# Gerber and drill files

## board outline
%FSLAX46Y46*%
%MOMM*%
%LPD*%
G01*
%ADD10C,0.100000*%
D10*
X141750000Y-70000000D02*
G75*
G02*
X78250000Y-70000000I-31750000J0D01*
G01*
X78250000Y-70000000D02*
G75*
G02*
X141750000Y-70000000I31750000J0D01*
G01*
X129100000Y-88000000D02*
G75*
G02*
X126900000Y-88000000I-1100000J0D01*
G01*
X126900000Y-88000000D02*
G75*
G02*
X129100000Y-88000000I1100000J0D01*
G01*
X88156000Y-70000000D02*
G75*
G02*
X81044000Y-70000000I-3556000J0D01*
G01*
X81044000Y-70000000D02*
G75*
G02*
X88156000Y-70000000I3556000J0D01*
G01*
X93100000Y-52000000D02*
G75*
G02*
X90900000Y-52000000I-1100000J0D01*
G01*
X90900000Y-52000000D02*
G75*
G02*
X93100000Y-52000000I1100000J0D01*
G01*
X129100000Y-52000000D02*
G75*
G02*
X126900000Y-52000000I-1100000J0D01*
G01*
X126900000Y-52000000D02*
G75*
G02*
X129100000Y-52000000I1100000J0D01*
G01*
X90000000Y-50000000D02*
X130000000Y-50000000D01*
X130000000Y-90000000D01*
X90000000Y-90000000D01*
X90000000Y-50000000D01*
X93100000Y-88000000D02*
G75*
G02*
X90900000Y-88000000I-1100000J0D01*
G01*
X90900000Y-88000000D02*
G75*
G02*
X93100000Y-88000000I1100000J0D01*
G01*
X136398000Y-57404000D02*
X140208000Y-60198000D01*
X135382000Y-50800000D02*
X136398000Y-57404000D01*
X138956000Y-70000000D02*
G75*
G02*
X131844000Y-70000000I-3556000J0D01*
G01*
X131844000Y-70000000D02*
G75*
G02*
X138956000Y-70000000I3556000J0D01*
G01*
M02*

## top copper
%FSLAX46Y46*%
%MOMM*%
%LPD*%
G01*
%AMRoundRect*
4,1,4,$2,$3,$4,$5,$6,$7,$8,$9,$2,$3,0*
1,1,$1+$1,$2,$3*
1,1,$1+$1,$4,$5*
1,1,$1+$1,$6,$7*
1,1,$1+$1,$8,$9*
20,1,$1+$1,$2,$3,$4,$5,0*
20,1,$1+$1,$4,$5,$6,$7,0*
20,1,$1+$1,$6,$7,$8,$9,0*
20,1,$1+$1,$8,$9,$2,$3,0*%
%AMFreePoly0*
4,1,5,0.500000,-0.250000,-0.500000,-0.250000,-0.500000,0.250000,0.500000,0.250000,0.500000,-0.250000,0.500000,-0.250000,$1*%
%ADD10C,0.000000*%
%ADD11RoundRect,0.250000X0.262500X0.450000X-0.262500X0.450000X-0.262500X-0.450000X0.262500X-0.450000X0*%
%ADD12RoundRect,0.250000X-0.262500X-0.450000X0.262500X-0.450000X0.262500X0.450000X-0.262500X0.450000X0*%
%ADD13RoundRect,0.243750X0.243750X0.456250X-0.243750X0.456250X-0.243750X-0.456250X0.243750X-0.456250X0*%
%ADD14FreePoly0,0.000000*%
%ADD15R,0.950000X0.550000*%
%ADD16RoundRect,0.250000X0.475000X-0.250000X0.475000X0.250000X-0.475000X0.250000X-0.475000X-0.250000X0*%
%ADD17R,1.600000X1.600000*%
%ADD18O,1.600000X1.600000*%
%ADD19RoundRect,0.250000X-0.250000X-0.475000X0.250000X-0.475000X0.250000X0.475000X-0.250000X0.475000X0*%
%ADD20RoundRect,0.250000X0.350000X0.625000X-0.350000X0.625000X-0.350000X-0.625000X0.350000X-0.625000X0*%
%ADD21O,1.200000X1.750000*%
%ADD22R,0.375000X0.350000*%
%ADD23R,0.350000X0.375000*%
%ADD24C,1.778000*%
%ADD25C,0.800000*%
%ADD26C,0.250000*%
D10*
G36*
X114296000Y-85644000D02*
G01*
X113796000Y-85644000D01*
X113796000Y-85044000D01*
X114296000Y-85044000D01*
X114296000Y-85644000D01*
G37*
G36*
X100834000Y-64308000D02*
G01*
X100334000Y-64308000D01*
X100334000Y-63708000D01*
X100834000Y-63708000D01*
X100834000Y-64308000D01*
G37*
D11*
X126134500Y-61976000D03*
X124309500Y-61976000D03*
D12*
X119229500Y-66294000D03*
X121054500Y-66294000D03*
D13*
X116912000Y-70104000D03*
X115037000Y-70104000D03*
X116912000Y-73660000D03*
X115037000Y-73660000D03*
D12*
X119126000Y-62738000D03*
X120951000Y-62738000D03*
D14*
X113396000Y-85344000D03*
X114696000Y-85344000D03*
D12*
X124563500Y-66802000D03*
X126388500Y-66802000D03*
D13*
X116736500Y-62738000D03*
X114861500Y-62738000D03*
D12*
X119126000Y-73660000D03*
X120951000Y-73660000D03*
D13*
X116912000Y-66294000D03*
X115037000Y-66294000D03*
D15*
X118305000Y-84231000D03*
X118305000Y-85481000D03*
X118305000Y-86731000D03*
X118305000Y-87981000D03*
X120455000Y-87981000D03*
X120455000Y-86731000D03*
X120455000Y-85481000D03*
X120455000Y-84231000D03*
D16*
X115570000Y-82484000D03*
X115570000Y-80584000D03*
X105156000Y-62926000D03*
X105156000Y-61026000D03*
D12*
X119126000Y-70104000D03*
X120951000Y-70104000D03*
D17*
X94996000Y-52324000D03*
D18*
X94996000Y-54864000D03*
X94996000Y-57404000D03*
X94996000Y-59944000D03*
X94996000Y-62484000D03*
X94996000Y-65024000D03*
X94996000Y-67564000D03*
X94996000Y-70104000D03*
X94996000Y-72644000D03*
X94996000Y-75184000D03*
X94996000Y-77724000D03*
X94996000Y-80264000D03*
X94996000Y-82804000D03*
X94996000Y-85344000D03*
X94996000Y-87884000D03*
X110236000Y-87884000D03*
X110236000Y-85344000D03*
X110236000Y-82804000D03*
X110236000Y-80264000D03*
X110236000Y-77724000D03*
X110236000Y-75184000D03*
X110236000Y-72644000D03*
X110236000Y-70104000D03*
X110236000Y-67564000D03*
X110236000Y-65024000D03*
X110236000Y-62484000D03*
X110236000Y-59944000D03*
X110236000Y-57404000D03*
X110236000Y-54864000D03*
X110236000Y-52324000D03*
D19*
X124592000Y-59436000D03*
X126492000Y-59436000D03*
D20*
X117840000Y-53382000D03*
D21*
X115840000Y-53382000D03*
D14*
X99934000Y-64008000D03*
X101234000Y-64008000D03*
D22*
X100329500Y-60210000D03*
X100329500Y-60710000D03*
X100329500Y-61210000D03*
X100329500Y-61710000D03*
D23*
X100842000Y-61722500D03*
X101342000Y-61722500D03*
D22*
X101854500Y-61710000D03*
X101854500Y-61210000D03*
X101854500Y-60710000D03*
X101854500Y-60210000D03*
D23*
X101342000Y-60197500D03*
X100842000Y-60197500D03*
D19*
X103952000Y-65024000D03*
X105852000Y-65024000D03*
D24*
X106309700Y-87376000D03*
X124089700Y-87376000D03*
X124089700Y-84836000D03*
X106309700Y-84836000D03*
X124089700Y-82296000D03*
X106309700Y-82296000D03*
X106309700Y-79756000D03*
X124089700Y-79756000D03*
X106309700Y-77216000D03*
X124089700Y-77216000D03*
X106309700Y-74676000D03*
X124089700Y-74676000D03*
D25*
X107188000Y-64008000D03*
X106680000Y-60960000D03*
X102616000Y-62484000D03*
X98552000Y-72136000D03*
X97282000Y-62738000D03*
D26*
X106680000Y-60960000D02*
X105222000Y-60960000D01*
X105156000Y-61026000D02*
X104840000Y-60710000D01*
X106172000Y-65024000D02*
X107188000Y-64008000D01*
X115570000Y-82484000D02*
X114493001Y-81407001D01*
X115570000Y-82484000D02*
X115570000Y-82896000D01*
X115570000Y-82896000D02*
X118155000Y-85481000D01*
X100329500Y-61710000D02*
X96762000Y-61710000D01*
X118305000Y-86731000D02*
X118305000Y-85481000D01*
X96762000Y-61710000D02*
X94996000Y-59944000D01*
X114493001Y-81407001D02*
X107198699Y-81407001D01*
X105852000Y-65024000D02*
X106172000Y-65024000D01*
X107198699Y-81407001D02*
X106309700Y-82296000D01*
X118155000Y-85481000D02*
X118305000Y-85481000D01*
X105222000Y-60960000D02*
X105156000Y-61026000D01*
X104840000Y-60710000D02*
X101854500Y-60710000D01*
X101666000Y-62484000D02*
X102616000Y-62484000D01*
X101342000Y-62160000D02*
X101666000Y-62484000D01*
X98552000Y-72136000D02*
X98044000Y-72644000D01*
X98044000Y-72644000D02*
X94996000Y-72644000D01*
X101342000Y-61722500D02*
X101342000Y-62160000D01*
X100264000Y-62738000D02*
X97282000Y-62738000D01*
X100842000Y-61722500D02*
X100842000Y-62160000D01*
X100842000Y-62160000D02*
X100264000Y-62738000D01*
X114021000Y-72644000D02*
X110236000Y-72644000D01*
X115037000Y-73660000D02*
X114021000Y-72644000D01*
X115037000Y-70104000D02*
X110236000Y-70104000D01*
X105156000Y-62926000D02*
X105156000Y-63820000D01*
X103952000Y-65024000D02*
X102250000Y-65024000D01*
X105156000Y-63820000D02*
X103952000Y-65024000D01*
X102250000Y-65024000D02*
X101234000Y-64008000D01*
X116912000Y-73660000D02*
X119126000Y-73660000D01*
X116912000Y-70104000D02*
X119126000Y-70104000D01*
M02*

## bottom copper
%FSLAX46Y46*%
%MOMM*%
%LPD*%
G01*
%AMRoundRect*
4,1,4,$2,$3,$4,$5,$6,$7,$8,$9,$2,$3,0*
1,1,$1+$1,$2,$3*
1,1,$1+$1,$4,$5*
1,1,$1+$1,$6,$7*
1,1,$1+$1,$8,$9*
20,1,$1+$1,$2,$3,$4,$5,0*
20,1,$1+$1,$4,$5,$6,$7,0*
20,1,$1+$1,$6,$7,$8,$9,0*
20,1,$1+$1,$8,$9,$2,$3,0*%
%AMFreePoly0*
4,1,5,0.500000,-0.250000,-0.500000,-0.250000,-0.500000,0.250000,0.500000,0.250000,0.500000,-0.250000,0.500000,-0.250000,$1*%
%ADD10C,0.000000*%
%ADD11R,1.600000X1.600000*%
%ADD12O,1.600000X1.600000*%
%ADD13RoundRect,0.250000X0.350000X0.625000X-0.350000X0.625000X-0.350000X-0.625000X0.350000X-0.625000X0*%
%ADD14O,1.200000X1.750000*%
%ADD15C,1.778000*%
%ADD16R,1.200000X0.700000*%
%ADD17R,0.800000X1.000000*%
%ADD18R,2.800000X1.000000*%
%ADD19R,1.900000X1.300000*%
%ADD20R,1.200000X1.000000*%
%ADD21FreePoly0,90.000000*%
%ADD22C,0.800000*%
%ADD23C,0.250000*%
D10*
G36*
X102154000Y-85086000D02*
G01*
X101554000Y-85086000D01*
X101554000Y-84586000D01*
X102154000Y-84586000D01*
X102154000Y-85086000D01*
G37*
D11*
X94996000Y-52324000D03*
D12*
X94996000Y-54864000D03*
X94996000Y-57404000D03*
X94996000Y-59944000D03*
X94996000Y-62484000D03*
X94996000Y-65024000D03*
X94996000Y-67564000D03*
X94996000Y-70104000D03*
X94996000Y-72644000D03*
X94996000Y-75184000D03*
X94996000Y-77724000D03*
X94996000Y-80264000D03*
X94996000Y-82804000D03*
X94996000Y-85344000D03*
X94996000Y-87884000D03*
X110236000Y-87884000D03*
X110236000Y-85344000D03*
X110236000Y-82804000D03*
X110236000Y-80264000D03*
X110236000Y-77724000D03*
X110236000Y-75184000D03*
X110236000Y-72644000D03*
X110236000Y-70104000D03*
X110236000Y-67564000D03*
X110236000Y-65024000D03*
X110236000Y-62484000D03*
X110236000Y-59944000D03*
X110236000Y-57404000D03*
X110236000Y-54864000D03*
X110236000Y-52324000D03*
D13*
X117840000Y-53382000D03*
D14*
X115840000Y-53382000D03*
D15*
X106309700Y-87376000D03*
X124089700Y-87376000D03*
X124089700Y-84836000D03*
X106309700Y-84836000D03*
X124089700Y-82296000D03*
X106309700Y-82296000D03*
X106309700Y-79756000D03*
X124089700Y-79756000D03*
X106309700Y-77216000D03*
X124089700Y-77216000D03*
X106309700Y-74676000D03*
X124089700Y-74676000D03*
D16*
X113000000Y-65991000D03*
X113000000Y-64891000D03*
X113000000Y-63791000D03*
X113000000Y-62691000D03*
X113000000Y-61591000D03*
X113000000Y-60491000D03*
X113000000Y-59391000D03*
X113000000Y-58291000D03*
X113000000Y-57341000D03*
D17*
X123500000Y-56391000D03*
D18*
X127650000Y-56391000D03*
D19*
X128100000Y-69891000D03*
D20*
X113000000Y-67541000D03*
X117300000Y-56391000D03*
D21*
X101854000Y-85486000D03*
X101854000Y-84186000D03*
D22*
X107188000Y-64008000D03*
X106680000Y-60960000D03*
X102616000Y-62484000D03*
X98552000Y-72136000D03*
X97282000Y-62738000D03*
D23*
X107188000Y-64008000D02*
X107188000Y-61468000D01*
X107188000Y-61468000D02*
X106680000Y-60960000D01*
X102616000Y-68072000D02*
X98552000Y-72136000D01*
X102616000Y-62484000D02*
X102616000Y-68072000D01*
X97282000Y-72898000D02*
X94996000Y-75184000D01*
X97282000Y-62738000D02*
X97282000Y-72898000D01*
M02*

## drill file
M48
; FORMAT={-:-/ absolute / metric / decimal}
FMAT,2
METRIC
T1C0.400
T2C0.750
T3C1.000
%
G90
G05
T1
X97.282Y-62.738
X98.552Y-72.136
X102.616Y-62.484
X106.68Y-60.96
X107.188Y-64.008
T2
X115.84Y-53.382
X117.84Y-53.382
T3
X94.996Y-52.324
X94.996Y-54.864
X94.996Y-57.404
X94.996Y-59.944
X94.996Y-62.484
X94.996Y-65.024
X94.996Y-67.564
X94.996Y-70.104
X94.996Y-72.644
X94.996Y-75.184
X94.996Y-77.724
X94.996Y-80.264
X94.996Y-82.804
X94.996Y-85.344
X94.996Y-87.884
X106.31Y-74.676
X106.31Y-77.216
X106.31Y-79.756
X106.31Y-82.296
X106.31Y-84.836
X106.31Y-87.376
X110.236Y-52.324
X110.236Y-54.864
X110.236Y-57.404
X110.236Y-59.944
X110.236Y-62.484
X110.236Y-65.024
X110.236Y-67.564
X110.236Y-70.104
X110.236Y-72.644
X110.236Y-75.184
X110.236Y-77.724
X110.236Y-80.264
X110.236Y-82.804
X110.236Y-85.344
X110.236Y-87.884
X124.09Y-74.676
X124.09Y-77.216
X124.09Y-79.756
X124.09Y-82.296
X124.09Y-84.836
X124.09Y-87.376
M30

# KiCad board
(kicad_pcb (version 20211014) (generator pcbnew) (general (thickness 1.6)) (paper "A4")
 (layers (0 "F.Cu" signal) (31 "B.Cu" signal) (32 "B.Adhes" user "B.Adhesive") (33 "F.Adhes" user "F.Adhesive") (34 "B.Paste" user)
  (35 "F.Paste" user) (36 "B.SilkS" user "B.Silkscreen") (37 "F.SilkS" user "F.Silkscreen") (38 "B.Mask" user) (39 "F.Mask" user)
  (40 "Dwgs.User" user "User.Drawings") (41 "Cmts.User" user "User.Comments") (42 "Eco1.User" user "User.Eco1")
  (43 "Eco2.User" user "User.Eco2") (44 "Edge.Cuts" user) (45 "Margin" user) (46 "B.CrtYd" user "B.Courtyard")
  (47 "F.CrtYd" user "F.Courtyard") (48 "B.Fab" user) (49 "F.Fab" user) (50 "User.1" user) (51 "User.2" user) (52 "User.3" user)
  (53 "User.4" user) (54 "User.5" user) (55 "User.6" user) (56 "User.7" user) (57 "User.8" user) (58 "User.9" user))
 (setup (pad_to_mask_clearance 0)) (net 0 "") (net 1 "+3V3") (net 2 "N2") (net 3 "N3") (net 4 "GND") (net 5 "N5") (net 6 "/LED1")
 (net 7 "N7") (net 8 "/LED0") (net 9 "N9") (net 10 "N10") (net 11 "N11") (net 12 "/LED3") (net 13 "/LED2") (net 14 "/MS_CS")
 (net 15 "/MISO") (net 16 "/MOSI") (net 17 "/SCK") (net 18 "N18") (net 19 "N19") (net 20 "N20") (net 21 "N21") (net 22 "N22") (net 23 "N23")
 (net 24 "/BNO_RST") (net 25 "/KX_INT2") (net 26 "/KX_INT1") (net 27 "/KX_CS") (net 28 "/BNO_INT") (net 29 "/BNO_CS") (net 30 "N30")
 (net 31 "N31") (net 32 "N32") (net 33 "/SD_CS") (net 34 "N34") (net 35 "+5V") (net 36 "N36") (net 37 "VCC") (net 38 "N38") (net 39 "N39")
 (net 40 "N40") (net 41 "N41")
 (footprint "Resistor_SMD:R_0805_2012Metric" (layer "F.Cu") (at 125.222 61.976 180)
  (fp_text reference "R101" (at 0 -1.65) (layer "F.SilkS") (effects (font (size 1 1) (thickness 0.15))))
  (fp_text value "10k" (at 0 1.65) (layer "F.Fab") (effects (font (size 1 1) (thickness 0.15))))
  (pad "1" smd roundrect (at -0.9125 0 180) (size 1.025 1.4) (layers "F.Cu" "F.Paste" "F.Mask") (roundrect_rratio 0.243902) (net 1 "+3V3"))
  (pad "2" smd roundrect (at 0.9125 0 180) (size 1.025 1.4) (layers "F.Cu" "F.Paste" "F.Mask") (roundrect_rratio 0.243902) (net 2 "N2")))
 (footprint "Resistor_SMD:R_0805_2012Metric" (layer "F.Cu") (at 120.142 66.294)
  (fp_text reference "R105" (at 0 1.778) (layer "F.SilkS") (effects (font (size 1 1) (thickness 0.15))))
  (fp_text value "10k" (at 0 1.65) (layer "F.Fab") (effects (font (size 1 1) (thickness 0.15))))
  (pad "1" smd roundrect (at -0.9125 0) (size 1.025 1.4) (layers "F.Cu" "F.Paste" "F.Mask") (roundrect_rratio 0.243902) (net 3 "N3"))
  (pad "2" smd roundrect (at 0.9125 0) (size 1.025 1.4) (layers "F.Cu" "F.Paste" "F.Mask") (roundrect_rratio 0.243902) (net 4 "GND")))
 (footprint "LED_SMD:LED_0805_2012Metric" (layer "F.Cu") (at 115.9745 70.104 180)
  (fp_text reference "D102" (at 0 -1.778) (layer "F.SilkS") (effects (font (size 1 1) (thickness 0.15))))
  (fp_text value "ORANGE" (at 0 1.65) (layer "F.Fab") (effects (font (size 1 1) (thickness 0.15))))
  (pad "1" smd roundrect (at -0.9375 0 180) (size 0.975 1.4) (layers "F.Cu" "F.Paste" "F.Mask") (roundrect_rratio 0.25) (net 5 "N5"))
  (pad "2" smd roundrect (at 0.9375 0 180) (size 0.975 1.4) (layers "F.Cu" "F.Paste" "F.Mask") (roundrect_rratio 0.25) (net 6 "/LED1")))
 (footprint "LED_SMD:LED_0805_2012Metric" (layer "F.Cu") (at 115.9745 73.66 180)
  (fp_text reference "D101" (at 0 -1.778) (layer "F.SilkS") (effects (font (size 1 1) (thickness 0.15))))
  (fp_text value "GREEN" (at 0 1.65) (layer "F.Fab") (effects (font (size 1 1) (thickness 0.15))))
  (pad "1" smd roundrect (at -0.9375 0 180) (size 0.975 1.4) (layers "F.Cu" "F.Paste" "F.Mask") (roundrect_rratio 0.25) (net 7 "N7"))
  (pad "2" smd roundrect (at 0.9375 0 180) (size 0.975 1.4) (layers "F.Cu" "F.Paste" "F.Mask") (roundrect_rratio 0.25) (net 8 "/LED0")))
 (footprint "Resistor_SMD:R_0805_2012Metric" (layer "F.Cu") (at 120.0385 62.738)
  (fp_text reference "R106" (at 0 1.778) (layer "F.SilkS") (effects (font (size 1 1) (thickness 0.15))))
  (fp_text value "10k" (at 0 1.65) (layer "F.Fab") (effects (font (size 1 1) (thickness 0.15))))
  (pad "1" smd roundrect (at -0.9125 0) (size 1.025 1.4) (layers "F.Cu" "F.Paste" "F.Mask") (roundrect_rratio 0.243902) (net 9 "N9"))
  (pad "2" smd roundrect (at 0.9125 0) (size 1.025 1.4) (layers "F.Cu" "F.Paste" "F.Mask") (roundrect_rratio 0.243902) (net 4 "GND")))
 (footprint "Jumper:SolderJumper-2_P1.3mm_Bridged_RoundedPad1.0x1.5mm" (layer "F.Cu") (at 114.046 85.344)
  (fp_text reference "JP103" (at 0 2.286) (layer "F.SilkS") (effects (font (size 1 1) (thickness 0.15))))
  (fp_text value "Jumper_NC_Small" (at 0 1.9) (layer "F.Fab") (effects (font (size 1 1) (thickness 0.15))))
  (fp_poly (pts (xy 0.25 -0.3) (xy -0.25 -0.3) (xy -0.25 0.3) (xy 0.25 0.3)) (layer "F.Cu") (width 0) (fill solid))
  (pad "1" smd custom (at -0.65 0) (size 1 0.5) (layers "F.Cu" "F.Mask") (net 1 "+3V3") (zone_connect 2)
   (options (clearance outline) (anchor rect)) (primitives))
  (pad "2" smd custom (at 0.65 0) (size 1 0.5) (layers "F.Cu" "F.Mask") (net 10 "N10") (zone_connect 2)
   (options (clearance outline) (anchor rect)) (primitives)))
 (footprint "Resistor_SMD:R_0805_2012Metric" (layer "F.Cu") (at 125.476 66.802)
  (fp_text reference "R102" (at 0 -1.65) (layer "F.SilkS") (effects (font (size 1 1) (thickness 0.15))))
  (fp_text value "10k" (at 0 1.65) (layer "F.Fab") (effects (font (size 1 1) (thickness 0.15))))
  (pad "1" smd roundrect (at -0.9125 0) (size 1.025 1.4) (layers "F.Cu" "F.Paste" "F.Mask") (roundrect_rratio 0.243902) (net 1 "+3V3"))
  (pad "2" smd roundrect (at 0.9125 0) (size 1.025 1.4) (layers "F.Cu" "F.Paste" "F.Mask") (roundrect_rratio 0.243902) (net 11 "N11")))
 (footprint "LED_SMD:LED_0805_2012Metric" (layer "F.Cu") (at 115.799 62.738 180)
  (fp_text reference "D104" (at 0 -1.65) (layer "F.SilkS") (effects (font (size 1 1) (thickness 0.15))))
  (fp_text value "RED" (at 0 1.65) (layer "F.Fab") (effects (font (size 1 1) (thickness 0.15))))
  (pad "1" smd roundrect (at -0.9375 0 180) (size 0.975 1.4) (layers "F.Cu" "F.Paste" "F.Mask") (roundrect_rratio 0.25) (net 9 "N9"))
  (pad "2" smd roundrect (at 0.9375 0 180) (size 0.975 1.4) (layers "F.Cu" "F.Paste" "F.Mask") (roundrect_rratio 0.25) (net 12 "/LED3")))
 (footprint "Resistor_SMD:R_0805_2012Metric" (layer "F.Cu") (at 120.0385 73.66)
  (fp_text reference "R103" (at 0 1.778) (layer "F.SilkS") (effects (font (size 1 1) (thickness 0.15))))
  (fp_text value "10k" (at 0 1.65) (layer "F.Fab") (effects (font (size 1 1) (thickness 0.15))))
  (pad "1" smd roundrect (at -0.9125 0) (size 1.025 1.4) (layers "F.Cu" "F.Paste" "F.Mask") (roundrect_rratio 0.243902) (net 7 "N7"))
  (pad "2" smd roundrect (at 0.9125 0) (size 1.025 1.4) (layers "F.Cu" "F.Paste" "F.Mask") (roundrect_rratio 0.243902) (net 4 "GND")))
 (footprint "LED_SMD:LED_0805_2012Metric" (layer "F.Cu") (at 115.9745 66.294 180)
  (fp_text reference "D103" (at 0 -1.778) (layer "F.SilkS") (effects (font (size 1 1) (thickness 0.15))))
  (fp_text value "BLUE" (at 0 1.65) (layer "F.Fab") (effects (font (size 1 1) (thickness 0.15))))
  (pad "1" smd roundrect (at -0.9375 0 180) (size 0.975 1.4) (layers "F.Cu" "F.Paste" "F.Mask") (roundrect_rratio 0.25) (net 3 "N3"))
  (pad "2" smd roundrect (at 0.9375 0 180) (size 0.975 1.4) (layers "F.Cu" "F.Paste" "F.Mask") (roundrect_rratio 0.25) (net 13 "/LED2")))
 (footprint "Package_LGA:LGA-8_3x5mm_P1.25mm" (layer "F.Cu") (at 119.38 86.106)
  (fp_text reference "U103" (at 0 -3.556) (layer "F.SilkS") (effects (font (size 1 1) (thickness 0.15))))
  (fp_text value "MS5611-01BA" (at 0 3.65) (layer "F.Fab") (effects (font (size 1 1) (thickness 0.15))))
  (pad "1" smd rect (at -1.075 -1.875) (size 0.95 0.55) (layers "F.Cu" "F.Paste" "F.Mask") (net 10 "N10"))
  (pad "2" smd rect (at -1.075 -0.625) (size 0.95 0.55) (layers "F.Cu" "F.Paste" "F.Mask") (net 4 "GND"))
  (pad "3" smd rect (at -1.075 0.625) (size 0.95 0.55) (layers "F.Cu" "F.Paste" "F.Mask") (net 4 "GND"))
  (pad "4" smd rect (at -1.075 1.875) (size 0.95 0.55) (layers "F.Cu" "F.Paste" "F.Mask") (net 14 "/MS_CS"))
  (pad "5" smd rect (at 1.075 1.875) (size 0.95 0.55) (layers "F.Cu" "F.Paste" "F.Mask") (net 14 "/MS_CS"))
  (pad "6" smd rect (at 1.075 0.625) (size 0.95 0.55) (layers "F.Cu" "F.Paste" "F.Mask") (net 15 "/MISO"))
  (pad "7" smd rect (at 1.075 -0.625) (size 0.95 0.55) (layers "F.Cu" "F.Paste" "F.Mask") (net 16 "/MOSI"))
  (pad "8" smd rect (at 1.075 -1.875) (size 0.95 0.55) (layers "F.Cu" "F.Paste" "F.Mask") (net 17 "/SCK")))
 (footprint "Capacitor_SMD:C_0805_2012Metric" (layer "F.Cu") (at 115.57 81.534 90)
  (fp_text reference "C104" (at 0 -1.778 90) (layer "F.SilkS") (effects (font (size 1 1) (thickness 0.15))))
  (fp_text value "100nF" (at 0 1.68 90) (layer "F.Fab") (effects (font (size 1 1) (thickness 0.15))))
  (pad "1" smd roundrect (at -0.95 0 90) (size 1 1.45) (layers "F.Cu" "F.Paste" "F.Mask") (roundrect_rratio 0.25) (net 4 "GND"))
  (pad "2" smd roundrect (at 0.95 0 90) (size 1 1.45) (layers "F.Cu" "F.Paste" "F.Mask") (roundrect_rratio 0.25) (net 10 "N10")))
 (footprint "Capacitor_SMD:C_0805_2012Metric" (layer "F.Cu") (at 105.156 61.976 90)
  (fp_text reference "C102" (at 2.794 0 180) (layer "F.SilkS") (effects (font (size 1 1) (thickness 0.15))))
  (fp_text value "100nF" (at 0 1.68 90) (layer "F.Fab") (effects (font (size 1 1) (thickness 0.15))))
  (pad "1" smd roundrect (at -0.95 0 90) (size 1 1.45) (layers "F.Cu" "F.Paste" "F.Mask") (roundrect_rratio 0.25) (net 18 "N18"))
  (pad "2" smd roundrect (at 0.95 0 90) (size 1 1.45) (layers "F.Cu" "F.Paste" "F.Mask") (roundrect_rratio 0.25) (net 4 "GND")))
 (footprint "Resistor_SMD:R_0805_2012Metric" (layer "F.Cu") (at 120.0385 70.104)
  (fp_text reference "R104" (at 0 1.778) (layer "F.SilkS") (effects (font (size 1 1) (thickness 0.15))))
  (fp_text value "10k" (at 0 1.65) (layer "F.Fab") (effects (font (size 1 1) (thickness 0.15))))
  (pad "1" smd roundrect (at -0.9125 0) (size 1.025 1.4) (layers "F.Cu" "F.Paste" "F.Mask") (roundrect_rratio 0.243902) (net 5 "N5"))
  (pad "2" smd roundrect (at 0.9125 0) (size 1.025 1.4) (layers "F.Cu" "F.Paste" "F.Mask") (roundrect_rratio 0.243902) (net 4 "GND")))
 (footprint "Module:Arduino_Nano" (layer "F.Cu") (at 94.996 52.324)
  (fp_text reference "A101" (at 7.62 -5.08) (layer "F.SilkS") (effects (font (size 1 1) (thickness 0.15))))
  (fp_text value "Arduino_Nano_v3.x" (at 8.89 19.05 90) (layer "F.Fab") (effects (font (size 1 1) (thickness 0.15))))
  (pad "1" thru_hole rect (at 0 0) (size 1.6 1.6) (drill 1) (layers *.Cu *.Mask) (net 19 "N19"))
  (pad "2" thru_hole oval (at 0 2.54) (size 1.6 1.6) (drill 1) (layers *.Cu *.Mask) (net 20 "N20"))
  (pad "3" thru_hole oval (at 0 5.08) (size 1.6 1.6) (drill 1) (layers *.Cu *.Mask) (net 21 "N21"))
  (pad "4" thru_hole oval (at 0 7.62) (size 1.6 1.6) (drill 1) (layers *.Cu *.Mask) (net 4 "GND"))
  (pad "5" thru_hole oval (at 0 10.16) (size 1.6 1.6) (drill 1) (layers *.Cu *.Mask) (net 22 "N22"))
  (pad "6" thru_hole oval (at 0 12.7) (size 1.6 1.6) (drill 1) (layers *.Cu *.Mask) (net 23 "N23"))
  (pad "7" thru_hole oval (at 0 15.24) (size 1.6 1.6) (drill 1) (layers *.Cu *.Mask) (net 14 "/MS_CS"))
  (pad "8" thru_hole oval (at 0 17.78) (size 1.6 1.6) (drill 1) (layers *.Cu *.Mask) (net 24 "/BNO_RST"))
  (pad "9" thru_hole oval (at 0 20.32) (size 1.6 1.6) (drill 1) (layers *.Cu *.Mask) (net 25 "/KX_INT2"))
  (pad "10" thru_hole oval (at 0 22.86) (size 1.6 1.6) (drill 1) (layers *.Cu *.Mask) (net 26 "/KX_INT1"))
  (pad "11" thru_hole oval (at 0 25.4) (size 1.6 1.6) (drill 1) (layers *.Cu *.Mask) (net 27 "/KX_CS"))
  (pad "12" thru_hole oval (at 0 27.94) (size 1.6 1.6) (drill 1) (layers *.Cu *.Mask) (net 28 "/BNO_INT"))
  (pad "13" thru_hole oval (at 0 30.48) (size 1.6 1.6) (drill 1) (layers *.Cu *.Mask) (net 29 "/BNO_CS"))
  (pad "14" thru_hole oval (at 0 33.02) (size 1.6 1.6) (drill 1) (layers *.Cu *.Mask) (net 16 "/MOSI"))
  (pad "15" thru_hole oval (at 0 35.56) (size 1.6 1.6) (drill 1) (layers *.Cu *.Mask) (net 15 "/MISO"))
  (pad "16" thru_hole oval (at 15.24 35.56) (size 1.6 1.6) (drill 1) (layers *.Cu *.Mask) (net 17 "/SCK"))
  (pad "17" thru_hole oval (at 15.24 33.02) (size 1.6 1.6) (drill 1) (layers *.Cu *.Mask) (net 1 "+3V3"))
  (pad "18" thru_hole oval (at 15.24 30.48) (size 1.6 1.6) (drill 1) (layers *.Cu *.Mask) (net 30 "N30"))
  (pad "19" thru_hole oval (at 15.24 27.94) (size 1.6 1.6) (drill 1) (layers *.Cu *.Mask) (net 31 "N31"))
  (pad "20" thru_hole oval (at 15.24 25.4) (size 1.6 1.6) (drill 1) (layers *.Cu *.Mask) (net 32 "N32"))
  (pad "21" thru_hole oval (at 15.24 22.86) (size 1.6 1.6) (drill 1) (layers *.Cu *.Mask) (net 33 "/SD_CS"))
  (pad "22" thru_hole oval (at 15.24 20.32) (size 1.6 1.6) (drill 1) (layers *.Cu *.Mask) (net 8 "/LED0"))
  (pad "23" thru_hole oval (at 15.24 17.78) (size 1.6 1.6) (drill 1) (layers *.Cu *.Mask) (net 6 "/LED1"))
  (pad "24" thru_hole oval (at 15.24 15.24) (size 1.6 1.6) (drill 1) (layers *.Cu *.Mask) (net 13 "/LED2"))
  (pad "25" thru_hole oval (at 15.24 12.7) (size 1.6 1.6) (drill 1) (layers *.Cu *.Mask) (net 12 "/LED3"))
  (pad "26" thru_hole oval (at 15.24 10.16) (size 1.6 1.6) (drill 1) (layers *.Cu *.Mask) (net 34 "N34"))
  (pad "27" thru_hole oval (at 15.24 7.62) (size 1.6 1.6) (drill 1) (layers *.Cu *.Mask) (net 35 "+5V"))
  (pad "28" thru_hole oval (at 15.24 5.08) (size 1.6 1.6) (drill 1) (layers *.Cu *.Mask) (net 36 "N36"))
  (pad "29" thru_hole oval (at 15.24 2.54) (size 1.6 1.6) (drill 1) (layers *.Cu *.Mask) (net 4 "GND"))
  (pad "30" thru_hole oval (at 15.24 0) (size 1.6 1.6) (drill 1) (layers *.Cu *.Mask) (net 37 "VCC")))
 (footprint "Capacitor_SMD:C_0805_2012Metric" (layer "F.Cu") (at 125.542 59.436)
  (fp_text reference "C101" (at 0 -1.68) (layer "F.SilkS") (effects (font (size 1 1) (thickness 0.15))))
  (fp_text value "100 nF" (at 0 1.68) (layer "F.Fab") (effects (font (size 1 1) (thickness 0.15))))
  (pad "1" smd roundrect (at -0.95 0) (size 1 1.45) (layers "F.Cu" "F.Paste" "F.Mask") (roundrect_rratio 0.25) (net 4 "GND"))
  (pad "2" smd roundrect (at 0.95 0) (size 1 1.45) (layers "F.Cu" "F.Paste" "F.Mask") (roundrect_rratio 0.25) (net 1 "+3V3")))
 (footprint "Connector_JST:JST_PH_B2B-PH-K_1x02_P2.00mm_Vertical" (layer "F.Cu") (at 117.84 53.382 180)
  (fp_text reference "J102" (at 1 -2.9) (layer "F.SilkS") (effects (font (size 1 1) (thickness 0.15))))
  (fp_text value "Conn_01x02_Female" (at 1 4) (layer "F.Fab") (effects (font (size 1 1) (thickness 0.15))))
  (pad "1" thru_hole roundrect (at 0 0 180) (size 1.2 1.75) (drill 0.75) (layers *.Cu *.Mask) (roundrect_rratio 0.208333) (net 4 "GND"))
  (pad "2" thru_hole oval (at 2 0 180) (size 1.2 1.75) (drill 0.75) (layers *.Cu *.Mask) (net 37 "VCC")))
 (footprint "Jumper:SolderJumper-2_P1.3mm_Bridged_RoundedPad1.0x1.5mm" (layer "F.Cu") (at 100.584 64.008)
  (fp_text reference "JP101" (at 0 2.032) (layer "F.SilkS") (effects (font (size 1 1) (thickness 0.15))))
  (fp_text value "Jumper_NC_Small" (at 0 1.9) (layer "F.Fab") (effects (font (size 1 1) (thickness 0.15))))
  (fp_poly (pts (xy 0.25 -0.3) (xy -0.25 -0.3) (xy -0.25 0.3) (xy 0.25 0.3)) (layer "F.Cu") (width 0) (fill solid))
  (pad "1" smd custom (at -0.65 0) (size 1 0.5) (layers "F.Cu" "F.Mask") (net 1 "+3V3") (zone_connect 2)
   (options (clearance outline) (anchor rect)) (primitives))
  (pad "2" smd custom (at 0.65 0) (size 1 0.5) (layers "F.Cu" "F.Mask") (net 18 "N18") (zone_connect 2)
   (options (clearance outline) (anchor rect)) (primitives)))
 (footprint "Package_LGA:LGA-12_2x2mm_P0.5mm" (layer "F.Cu") (at 101.092 60.96)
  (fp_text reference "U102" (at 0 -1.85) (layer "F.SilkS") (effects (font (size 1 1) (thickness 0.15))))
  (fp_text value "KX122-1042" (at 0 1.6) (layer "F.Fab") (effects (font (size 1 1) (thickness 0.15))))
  (pad "1" smd rect (at -0.7625 -0.75) (size 0.375 0.35) (layers "F.Cu" "F.Paste" "F.Mask") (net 15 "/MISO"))
  (pad "2" smd rect (at -0.7625 -0.25) (size 0.375 0.35) (layers "F.Cu" "F.Paste" "F.Mask") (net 16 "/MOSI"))
  (pad "3" smd rect (at -0.7625 0.25) (size 0.375 0.35) (layers "F.Cu" "F.Paste" "F.Mask") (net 18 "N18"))
  (pad "4" smd rect (at -0.7625 0.75) (size 0.375 0.35) (layers "F.Cu" "F.Paste" "F.Mask") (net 4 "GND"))
  (pad "5" smd rect (at -0.25 0.7625 90) (size 0.375 0.35) (layers "F.Cu" "F.Paste" "F.Mask") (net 26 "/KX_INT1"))
  (pad "6" smd rect (at 0.25 0.7625 90) (size 0.375 0.35) (layers "F.Cu" "F.Paste" "F.Mask") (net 25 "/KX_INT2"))
  (pad "7" smd rect (at 0.7625 0.75) (size 0.375 0.35) (layers "F.Cu" "F.Paste" "F.Mask") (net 18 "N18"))
  (pad "8" smd rect (at 0.7625 0.25) (size 0.375 0.35) (layers "F.Cu" "F.Paste" "F.Mask"))
  (pad "9" smd rect (at 0.7625 -0.25) (size 0.375 0.35) (layers "F.Cu" "F.Paste" "F.Mask") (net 4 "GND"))
  (pad "10" smd rect (at 0.7625 -0.75) (size 0.375 0.35) (layers "F.Cu" "F.Paste" "F.Mask") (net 27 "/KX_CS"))
  (pad "11" smd rect (at 0.25 -0.7625 90) (size 0.375 0.35) (layers "F.Cu" "F.Paste" "F.Mask") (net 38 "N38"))
  (pad "12" smd rect (at -0.25 -0.7625 90) (size 0.375 0.35) (layers "F.Cu" "F.Paste" "F.Mask") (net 17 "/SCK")))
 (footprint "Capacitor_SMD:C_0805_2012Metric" (layer "F.Cu") (at 104.902 65.024)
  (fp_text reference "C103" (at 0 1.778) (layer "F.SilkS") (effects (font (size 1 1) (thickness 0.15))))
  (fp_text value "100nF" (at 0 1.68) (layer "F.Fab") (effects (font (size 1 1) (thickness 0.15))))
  (pad "1" smd roundrect (at -0.95 0) (size 1 1.45) (layers "F.Cu" "F.Paste" "F.Mask") (roundrect_rratio 0.25) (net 18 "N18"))
  (pad "2" smd roundrect (at 0.95 0) (size 1 1.45) (layers "F.Cu" "F.Paste" "F.Mask") (roundrect_rratio 0.25) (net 4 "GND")))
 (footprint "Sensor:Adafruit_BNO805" (layer "B.Cu") (at 98.7913 81.1276 90)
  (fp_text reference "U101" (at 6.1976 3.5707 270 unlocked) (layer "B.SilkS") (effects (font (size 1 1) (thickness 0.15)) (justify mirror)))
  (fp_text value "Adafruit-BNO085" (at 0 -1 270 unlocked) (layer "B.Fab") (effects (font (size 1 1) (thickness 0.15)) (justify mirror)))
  (pad "1" thru_hole circle (at -6.2484 7.5184) (size 1.778 1.778) (drill 1) (layers *.Cu *.Mask) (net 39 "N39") (solder_mask_margin 0.0508))
  (pad "1" thru_hole circle (at -6.2484 25.2984) (size 1.778 1.778) (drill 1) (layers *.Cu *.Mask) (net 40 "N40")
   (solder_mask_margin 0.0508))
  (pad "2" thru_hole circle (at -3.7084 25.2984) (size 1.778 1.778) (drill 1) (layers *.Cu *.Mask) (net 1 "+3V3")
   (solder_mask_margin 0.0508))
  (pad "2" thru_hole circle (at -3.7084 7.5184) (size 1.778 1.778) (drill 1) (layers *.Cu *.Mask) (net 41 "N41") (solder_mask_margin 0.0508))
  (pad "3" thru_hole circle (at -1.1684 25.2984) (size 1.778 1.778) (drill 1) (layers *.Cu *.Mask) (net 1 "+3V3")
   (solder_mask_margin 0.0508))
  (pad "3" thru_hole circle (at -1.1684 7.5184) (size 1.778 1.778) (drill 1) (layers *.Cu *.Mask) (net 4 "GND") (solder_mask_margin 0.0508))
  (pad "4" thru_hole circle (at 1.3716 7.5184) (size 1.778 1.778) (drill 1) (layers *.Cu *.Mask) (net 17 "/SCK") (solder_mask_margin 0.0508))
  (pad "4" thru_hole circle (at 1.3716 25.2984) (size 1.778 1.778) (drill 1) (layers *.Cu *.Mask) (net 24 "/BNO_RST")
   (solder_mask_margin 0.0508))
  (pad "5" thru_hole circle (at 3.9116 7.5184) (size 1.778 1.778) (drill 1) (layers *.Cu *.Mask) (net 15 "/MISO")
   (solder_mask_margin 0.0508))
  (pad "5" thru_hole circle (at 3.9116 25.2984) (size 1.778 1.778) (drill 1) (layers *.Cu *.Mask) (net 16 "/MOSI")
   (solder_mask_margin 0.0508))
  (pad "6" thru_hole circle (at 6.4516 7.5184) (size 1.778 1.778) (drill 1) (layers *.Cu *.Mask) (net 28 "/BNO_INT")
   (solder_mask_margin 0.0508))
  (pad "6" thru_hole circle (at 6.4516 25.2984) (size 1.778 1.778) (drill 1) (layers *.Cu *.Mask) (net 29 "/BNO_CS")
   (solder_mask_margin 0.0508)))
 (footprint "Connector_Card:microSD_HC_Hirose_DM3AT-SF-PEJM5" (layer "B.Cu") (at 120.725 63.216 -90)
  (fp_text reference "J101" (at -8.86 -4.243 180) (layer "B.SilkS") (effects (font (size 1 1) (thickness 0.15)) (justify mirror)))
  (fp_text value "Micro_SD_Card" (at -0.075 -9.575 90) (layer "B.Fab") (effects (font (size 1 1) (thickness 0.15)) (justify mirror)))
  (pad "1" smd rect (at 2.775 7.725 270) (size 0.7 1.2) (layers "B.Cu" "B.Paste" "B.Mask") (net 11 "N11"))
  (pad "2" smd rect (at 1.675 7.725 270) (size 0.7 1.2) (layers "B.Cu" "B.Paste" "B.Mask") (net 33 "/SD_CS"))
  (pad "3" smd rect (at 0.575 7.725 270) (size 0.7 1.2) (layers "B.Cu" "B.Paste" "B.Mask") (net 16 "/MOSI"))
  (pad "4" smd rect (at -0.525 7.725 270) (size 0.7 1.2) (layers "B.Cu" "B.Paste" "B.Mask") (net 1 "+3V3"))
  (pad "5" smd rect (at -1.625 7.725 270) (size 0.7 1.2) (layers "B.Cu" "B.Paste" "B.Mask") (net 17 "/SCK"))
  (pad "6" smd rect (at -2.725 7.725 270) (size 0.7 1.2) (layers "B.Cu" "B.Paste" "B.Mask") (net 4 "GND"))
  (pad "7" smd rect (at -3.825 7.725 270) (size 0.7 1.2) (layers "B.Cu" "B.Paste" "B.Mask") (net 15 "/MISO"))
  (pad "8" smd rect (at -4.925 7.725 270) (size 0.7 1.2) (layers "B.Cu" "B.Paste" "B.Mask") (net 2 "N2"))
  (pad "9" smd rect (at -5.875 7.725 270) (size 0.7 1.2) (layers "B.Cu" "B.Paste" "B.Mask") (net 4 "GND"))
  (pad "10" smd rect (at -6.825 -2.775 270) (size 1 0.8) (layers "B.Cu" "B.Paste" "B.Mask"))
  (pad "11" smd rect (at -6.825 -6.925 270) (size 1 2.8) (layers "B.Cu" "B.Paste" "B.Mask"))
  (pad "11" smd rect (at 6.675 -7.375 270) (size 1.3 1.9) (layers "B.Cu" "B.Paste" "B.Mask"))
  (pad "11" smd rect (at 4.325 7.725 270) (size 1 1.2) (layers "B.Cu" "B.Paste" "B.Mask"))
  (pad "11" smd rect (at -6.825 3.425 270) (size 1 1.2) (layers "B.Cu" "B.Paste" "B.Mask"))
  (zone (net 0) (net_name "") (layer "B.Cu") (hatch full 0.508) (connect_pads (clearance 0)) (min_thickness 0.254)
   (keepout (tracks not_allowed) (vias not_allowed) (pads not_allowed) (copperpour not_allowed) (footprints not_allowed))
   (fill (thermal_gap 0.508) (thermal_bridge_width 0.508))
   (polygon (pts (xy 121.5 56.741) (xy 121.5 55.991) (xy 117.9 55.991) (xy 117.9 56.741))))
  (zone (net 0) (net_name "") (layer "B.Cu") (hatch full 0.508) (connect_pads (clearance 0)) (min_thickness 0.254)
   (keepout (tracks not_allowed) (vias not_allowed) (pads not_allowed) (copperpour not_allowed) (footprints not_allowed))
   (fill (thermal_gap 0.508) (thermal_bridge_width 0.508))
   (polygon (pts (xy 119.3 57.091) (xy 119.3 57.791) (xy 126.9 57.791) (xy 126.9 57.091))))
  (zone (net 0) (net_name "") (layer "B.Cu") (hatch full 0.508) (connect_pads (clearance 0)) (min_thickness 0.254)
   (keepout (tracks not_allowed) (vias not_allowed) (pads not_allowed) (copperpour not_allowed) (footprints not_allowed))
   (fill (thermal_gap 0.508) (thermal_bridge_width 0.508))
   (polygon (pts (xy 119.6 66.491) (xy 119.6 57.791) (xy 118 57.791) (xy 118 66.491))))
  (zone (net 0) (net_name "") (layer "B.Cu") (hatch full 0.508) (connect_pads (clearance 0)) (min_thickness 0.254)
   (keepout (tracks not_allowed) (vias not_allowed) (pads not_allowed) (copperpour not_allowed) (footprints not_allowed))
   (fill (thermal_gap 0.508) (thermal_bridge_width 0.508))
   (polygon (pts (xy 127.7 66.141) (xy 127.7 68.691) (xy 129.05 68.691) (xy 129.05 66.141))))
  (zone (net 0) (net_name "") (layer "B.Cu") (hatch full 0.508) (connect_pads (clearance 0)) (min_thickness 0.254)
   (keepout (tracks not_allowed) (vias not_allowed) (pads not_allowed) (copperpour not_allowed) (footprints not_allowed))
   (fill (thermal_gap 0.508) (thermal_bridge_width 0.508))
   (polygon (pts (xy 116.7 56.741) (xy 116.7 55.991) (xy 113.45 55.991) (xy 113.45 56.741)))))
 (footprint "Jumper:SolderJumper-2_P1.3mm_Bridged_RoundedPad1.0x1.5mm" (layer "B.Cu") (at 101.854 84.836 90)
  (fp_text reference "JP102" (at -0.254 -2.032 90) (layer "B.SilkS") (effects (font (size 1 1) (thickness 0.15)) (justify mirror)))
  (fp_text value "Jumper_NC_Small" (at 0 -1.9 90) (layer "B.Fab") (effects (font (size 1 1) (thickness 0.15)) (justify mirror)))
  (fp_poly (pts (xy 0.25 0.3) (xy -0.25 0.3) (xy -0.25 -0.3) (xy 0.25 -0.3)) (layer "B.Cu") (width 0) (fill solid))
  (pad "1" smd custom (at -0.65 0 90) (size 1 0.5) (layers "B.Cu" "B.Mask") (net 39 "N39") (zone_connect 2)
   (options (clearance outline) (anchor rect)) (primitives))
  (pad "2" smd custom (at 0.65 0 90) (size 1 0.5) (layers "B.Cu" "B.Mask") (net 1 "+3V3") (zone_connect 2)
   (options (clearance outline) (anchor rect)) (primitives)))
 (gr_circle (center 110 70) (end 141.75 70) (layer "Edge.Cuts") (width 0.1) (fill none))
 (gr_circle (center 128 88) (end 129.1 88) (layer "Edge.Cuts") (width 0.1) (fill none))
 (gr_circle (center 84.6 70) (end 88.156 70) (layer "Edge.Cuts") (width 0.1) (fill none))
 (gr_circle (center 92 52) (end 93.1 52) (layer "Edge.Cuts") (width 0.1) (fill none))
 (gr_circle (center 128 52) (end 129.1 52) (layer "Edge.Cuts") (width 0.1) (fill none))
 (gr_rect (start 90 50) (end 130 90) (layer "Edge.Cuts") (width 0.1) (fill none))
 (gr_circle (center 92 88) (end 93.1 88) (layer "Edge.Cuts") (width 0.1) (fill none))
 (gr_line (start 136.398 57.404) (end 140.208 60.198) (layer "Edge.Cuts") (width 0.1))
 (gr_line (start 135.382 50.8) (end 136.398 57.404) (layer "Edge.Cuts") (width 0.1))
 (gr_circle (center 135.4 70) (end 138.956 70) (layer "Edge.Cuts") (width 0.1) (fill none))
 (segment (start 106.68 60.96) (end 105.222 60.96) (width 0.25) (layer "F.Cu") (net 4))
 (segment (start 105.156 61.026) (end 104.84 60.71) (width 0.25) (layer "F.Cu") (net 4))
 (segment (start 106.172 65.024) (end 107.188 64.008) (width 0.25) (layer "F.Cu") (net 4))
 (segment (start 115.57 82.484) (end 114.493001 81.407001) (width 0.25) (layer "F.Cu") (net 4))
 (segment (start 115.57 82.484) (end 115.57 82.896) (width 0.25) (layer "F.Cu") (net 4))
 (segment (start 115.57 82.896) (end 118.155 85.481) (width 0.25) (layer "F.Cu") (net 4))
 (segment (start 100.3295 61.71) (end 96.762 61.71) (width 0.25) (layer "F.Cu") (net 4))
 (segment (start 118.305 86.731) (end 118.305 85.481) (width 0.25) (layer "F.Cu") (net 4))
 (segment (start 96.762 61.71) (end 94.996 59.944) (width 0.25) (layer "F.Cu") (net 4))
 (segment (start 114.493001 81.407001) (end 107.198699 81.407001) (width 0.25) (layer "F.Cu") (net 4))
 (segment (start 105.852 65.024) (end 106.172 65.024) (width 0.25) (layer "F.Cu") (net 4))
 (segment (start 107.198699 81.407001) (end 106.3097 82.296) (width 0.25) (layer "F.Cu") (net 4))
 (segment (start 118.155 85.481) (end 118.305 85.481) (width 0.25) (layer "F.Cu") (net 4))
 (segment (start 105.222 60.96) (end 105.156 61.026) (width 0.25) (layer "F.Cu") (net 4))
 (segment (start 104.84 60.71) (end 101.8545 60.71) (width 0.25) (layer "F.Cu") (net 4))
 (via (at 107.188 64.008) (size 0.8) (drill 0.4) (layers "F.Cu" "B.Cu") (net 4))
 (via (at 106.68 60.96) (size 0.8) (drill 0.4) (layers "F.Cu" "B.Cu") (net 4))
 (segment (start 107.188 64.008) (end 107.188 61.468) (width 0.25) (layer "B.Cu") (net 4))
 (segment (start 107.188 61.468) (end 106.68 60.96) (width 0.25) (layer "B.Cu") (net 4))
 (segment (start 101.666 62.484) (end 102.616 62.484) (width 0.25) (layer "F.Cu") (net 25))
 (segment (start 101.342 62.16) (end 101.666 62.484) (width 0.25) (layer "F.Cu") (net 25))
 (segment (start 98.552 72.136) (end 98.044 72.644) (width 0.25) (layer "F.Cu") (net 25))
 (segment (start 98.044 72.644) (end 94.996 72.644) (width 0.25) (layer "F.Cu") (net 25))
 (segment (start 101.342 61.7225) (end 101.342 62.16) (width 0.25) (layer "F.Cu") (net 25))
 (via (at 102.616 62.484) (size 0.8) (drill 0.4) (layers "F.Cu" "B.Cu") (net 25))
 (via (at 98.552 72.136) (size 0.8) (drill 0.4) (layers "F.Cu" "B.Cu") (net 25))
 (segment (start 102.616 68.072) (end 98.552 72.136) (width 0.25) (layer "B.Cu") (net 25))
 (segment (start 102.616 62.484) (end 102.616 68.072) (width 0.25) (layer "B.Cu") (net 25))
 (segment (start 100.264 62.738) (end 97.282 62.738) (width 0.25) (layer "F.Cu") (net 26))
 (segment (start 100.842 61.7225) (end 100.842 62.16) (width 0.25) (layer "F.Cu") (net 26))
 (segment (start 100.842 62.16) (end 100.264 62.738) (width 0.25) (layer "F.Cu") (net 26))
 (via (at 97.282 62.738) (size 0.8) (drill 0.4) (layers "F.Cu" "B.Cu") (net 26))
 (segment (start 97.282 72.898) (end 94.996 75.184) (width 0.25) (layer "B.Cu") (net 26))
 (segment (start 97.282 62.738) (end 97.282 72.898) (width 0.25) (layer "B.Cu") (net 26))
 (segment (start 114.021 72.644) (end 110.236 72.644) (width 0.25) (layer "F.Cu") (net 8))
 (segment (start 115.037 73.66) (end 114.021 72.644) (width 0.25) (layer "F.Cu") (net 8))
 (segment (start 115.037 70.104) (end 110.236 70.104) (width 0.25) (layer "F.Cu") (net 6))
 (segment (start 105.156 62.926) (end 105.156 63.82) (width 0.25) (layer "F.Cu") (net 18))
 (segment (start 103.952 65.024) (end 102.25 65.024) (width 0.25) (layer "F.Cu") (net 18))
 (segment (start 105.156 63.82) (end 103.952 65.024) (width 0.25) (layer "F.Cu") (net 18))
 (segment (start 102.25 65.024) (end 101.234 64.008) (width 0.25) (layer "F.Cu") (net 18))
 (segment (start 116.912 73.66) (end 119.126 73.66) (width 0.25) (layer "F.Cu") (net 7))
 (segment (start 116.912 70.104) (end 119.126 70.104) (width 0.25) (layer "F.Cu") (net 5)))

